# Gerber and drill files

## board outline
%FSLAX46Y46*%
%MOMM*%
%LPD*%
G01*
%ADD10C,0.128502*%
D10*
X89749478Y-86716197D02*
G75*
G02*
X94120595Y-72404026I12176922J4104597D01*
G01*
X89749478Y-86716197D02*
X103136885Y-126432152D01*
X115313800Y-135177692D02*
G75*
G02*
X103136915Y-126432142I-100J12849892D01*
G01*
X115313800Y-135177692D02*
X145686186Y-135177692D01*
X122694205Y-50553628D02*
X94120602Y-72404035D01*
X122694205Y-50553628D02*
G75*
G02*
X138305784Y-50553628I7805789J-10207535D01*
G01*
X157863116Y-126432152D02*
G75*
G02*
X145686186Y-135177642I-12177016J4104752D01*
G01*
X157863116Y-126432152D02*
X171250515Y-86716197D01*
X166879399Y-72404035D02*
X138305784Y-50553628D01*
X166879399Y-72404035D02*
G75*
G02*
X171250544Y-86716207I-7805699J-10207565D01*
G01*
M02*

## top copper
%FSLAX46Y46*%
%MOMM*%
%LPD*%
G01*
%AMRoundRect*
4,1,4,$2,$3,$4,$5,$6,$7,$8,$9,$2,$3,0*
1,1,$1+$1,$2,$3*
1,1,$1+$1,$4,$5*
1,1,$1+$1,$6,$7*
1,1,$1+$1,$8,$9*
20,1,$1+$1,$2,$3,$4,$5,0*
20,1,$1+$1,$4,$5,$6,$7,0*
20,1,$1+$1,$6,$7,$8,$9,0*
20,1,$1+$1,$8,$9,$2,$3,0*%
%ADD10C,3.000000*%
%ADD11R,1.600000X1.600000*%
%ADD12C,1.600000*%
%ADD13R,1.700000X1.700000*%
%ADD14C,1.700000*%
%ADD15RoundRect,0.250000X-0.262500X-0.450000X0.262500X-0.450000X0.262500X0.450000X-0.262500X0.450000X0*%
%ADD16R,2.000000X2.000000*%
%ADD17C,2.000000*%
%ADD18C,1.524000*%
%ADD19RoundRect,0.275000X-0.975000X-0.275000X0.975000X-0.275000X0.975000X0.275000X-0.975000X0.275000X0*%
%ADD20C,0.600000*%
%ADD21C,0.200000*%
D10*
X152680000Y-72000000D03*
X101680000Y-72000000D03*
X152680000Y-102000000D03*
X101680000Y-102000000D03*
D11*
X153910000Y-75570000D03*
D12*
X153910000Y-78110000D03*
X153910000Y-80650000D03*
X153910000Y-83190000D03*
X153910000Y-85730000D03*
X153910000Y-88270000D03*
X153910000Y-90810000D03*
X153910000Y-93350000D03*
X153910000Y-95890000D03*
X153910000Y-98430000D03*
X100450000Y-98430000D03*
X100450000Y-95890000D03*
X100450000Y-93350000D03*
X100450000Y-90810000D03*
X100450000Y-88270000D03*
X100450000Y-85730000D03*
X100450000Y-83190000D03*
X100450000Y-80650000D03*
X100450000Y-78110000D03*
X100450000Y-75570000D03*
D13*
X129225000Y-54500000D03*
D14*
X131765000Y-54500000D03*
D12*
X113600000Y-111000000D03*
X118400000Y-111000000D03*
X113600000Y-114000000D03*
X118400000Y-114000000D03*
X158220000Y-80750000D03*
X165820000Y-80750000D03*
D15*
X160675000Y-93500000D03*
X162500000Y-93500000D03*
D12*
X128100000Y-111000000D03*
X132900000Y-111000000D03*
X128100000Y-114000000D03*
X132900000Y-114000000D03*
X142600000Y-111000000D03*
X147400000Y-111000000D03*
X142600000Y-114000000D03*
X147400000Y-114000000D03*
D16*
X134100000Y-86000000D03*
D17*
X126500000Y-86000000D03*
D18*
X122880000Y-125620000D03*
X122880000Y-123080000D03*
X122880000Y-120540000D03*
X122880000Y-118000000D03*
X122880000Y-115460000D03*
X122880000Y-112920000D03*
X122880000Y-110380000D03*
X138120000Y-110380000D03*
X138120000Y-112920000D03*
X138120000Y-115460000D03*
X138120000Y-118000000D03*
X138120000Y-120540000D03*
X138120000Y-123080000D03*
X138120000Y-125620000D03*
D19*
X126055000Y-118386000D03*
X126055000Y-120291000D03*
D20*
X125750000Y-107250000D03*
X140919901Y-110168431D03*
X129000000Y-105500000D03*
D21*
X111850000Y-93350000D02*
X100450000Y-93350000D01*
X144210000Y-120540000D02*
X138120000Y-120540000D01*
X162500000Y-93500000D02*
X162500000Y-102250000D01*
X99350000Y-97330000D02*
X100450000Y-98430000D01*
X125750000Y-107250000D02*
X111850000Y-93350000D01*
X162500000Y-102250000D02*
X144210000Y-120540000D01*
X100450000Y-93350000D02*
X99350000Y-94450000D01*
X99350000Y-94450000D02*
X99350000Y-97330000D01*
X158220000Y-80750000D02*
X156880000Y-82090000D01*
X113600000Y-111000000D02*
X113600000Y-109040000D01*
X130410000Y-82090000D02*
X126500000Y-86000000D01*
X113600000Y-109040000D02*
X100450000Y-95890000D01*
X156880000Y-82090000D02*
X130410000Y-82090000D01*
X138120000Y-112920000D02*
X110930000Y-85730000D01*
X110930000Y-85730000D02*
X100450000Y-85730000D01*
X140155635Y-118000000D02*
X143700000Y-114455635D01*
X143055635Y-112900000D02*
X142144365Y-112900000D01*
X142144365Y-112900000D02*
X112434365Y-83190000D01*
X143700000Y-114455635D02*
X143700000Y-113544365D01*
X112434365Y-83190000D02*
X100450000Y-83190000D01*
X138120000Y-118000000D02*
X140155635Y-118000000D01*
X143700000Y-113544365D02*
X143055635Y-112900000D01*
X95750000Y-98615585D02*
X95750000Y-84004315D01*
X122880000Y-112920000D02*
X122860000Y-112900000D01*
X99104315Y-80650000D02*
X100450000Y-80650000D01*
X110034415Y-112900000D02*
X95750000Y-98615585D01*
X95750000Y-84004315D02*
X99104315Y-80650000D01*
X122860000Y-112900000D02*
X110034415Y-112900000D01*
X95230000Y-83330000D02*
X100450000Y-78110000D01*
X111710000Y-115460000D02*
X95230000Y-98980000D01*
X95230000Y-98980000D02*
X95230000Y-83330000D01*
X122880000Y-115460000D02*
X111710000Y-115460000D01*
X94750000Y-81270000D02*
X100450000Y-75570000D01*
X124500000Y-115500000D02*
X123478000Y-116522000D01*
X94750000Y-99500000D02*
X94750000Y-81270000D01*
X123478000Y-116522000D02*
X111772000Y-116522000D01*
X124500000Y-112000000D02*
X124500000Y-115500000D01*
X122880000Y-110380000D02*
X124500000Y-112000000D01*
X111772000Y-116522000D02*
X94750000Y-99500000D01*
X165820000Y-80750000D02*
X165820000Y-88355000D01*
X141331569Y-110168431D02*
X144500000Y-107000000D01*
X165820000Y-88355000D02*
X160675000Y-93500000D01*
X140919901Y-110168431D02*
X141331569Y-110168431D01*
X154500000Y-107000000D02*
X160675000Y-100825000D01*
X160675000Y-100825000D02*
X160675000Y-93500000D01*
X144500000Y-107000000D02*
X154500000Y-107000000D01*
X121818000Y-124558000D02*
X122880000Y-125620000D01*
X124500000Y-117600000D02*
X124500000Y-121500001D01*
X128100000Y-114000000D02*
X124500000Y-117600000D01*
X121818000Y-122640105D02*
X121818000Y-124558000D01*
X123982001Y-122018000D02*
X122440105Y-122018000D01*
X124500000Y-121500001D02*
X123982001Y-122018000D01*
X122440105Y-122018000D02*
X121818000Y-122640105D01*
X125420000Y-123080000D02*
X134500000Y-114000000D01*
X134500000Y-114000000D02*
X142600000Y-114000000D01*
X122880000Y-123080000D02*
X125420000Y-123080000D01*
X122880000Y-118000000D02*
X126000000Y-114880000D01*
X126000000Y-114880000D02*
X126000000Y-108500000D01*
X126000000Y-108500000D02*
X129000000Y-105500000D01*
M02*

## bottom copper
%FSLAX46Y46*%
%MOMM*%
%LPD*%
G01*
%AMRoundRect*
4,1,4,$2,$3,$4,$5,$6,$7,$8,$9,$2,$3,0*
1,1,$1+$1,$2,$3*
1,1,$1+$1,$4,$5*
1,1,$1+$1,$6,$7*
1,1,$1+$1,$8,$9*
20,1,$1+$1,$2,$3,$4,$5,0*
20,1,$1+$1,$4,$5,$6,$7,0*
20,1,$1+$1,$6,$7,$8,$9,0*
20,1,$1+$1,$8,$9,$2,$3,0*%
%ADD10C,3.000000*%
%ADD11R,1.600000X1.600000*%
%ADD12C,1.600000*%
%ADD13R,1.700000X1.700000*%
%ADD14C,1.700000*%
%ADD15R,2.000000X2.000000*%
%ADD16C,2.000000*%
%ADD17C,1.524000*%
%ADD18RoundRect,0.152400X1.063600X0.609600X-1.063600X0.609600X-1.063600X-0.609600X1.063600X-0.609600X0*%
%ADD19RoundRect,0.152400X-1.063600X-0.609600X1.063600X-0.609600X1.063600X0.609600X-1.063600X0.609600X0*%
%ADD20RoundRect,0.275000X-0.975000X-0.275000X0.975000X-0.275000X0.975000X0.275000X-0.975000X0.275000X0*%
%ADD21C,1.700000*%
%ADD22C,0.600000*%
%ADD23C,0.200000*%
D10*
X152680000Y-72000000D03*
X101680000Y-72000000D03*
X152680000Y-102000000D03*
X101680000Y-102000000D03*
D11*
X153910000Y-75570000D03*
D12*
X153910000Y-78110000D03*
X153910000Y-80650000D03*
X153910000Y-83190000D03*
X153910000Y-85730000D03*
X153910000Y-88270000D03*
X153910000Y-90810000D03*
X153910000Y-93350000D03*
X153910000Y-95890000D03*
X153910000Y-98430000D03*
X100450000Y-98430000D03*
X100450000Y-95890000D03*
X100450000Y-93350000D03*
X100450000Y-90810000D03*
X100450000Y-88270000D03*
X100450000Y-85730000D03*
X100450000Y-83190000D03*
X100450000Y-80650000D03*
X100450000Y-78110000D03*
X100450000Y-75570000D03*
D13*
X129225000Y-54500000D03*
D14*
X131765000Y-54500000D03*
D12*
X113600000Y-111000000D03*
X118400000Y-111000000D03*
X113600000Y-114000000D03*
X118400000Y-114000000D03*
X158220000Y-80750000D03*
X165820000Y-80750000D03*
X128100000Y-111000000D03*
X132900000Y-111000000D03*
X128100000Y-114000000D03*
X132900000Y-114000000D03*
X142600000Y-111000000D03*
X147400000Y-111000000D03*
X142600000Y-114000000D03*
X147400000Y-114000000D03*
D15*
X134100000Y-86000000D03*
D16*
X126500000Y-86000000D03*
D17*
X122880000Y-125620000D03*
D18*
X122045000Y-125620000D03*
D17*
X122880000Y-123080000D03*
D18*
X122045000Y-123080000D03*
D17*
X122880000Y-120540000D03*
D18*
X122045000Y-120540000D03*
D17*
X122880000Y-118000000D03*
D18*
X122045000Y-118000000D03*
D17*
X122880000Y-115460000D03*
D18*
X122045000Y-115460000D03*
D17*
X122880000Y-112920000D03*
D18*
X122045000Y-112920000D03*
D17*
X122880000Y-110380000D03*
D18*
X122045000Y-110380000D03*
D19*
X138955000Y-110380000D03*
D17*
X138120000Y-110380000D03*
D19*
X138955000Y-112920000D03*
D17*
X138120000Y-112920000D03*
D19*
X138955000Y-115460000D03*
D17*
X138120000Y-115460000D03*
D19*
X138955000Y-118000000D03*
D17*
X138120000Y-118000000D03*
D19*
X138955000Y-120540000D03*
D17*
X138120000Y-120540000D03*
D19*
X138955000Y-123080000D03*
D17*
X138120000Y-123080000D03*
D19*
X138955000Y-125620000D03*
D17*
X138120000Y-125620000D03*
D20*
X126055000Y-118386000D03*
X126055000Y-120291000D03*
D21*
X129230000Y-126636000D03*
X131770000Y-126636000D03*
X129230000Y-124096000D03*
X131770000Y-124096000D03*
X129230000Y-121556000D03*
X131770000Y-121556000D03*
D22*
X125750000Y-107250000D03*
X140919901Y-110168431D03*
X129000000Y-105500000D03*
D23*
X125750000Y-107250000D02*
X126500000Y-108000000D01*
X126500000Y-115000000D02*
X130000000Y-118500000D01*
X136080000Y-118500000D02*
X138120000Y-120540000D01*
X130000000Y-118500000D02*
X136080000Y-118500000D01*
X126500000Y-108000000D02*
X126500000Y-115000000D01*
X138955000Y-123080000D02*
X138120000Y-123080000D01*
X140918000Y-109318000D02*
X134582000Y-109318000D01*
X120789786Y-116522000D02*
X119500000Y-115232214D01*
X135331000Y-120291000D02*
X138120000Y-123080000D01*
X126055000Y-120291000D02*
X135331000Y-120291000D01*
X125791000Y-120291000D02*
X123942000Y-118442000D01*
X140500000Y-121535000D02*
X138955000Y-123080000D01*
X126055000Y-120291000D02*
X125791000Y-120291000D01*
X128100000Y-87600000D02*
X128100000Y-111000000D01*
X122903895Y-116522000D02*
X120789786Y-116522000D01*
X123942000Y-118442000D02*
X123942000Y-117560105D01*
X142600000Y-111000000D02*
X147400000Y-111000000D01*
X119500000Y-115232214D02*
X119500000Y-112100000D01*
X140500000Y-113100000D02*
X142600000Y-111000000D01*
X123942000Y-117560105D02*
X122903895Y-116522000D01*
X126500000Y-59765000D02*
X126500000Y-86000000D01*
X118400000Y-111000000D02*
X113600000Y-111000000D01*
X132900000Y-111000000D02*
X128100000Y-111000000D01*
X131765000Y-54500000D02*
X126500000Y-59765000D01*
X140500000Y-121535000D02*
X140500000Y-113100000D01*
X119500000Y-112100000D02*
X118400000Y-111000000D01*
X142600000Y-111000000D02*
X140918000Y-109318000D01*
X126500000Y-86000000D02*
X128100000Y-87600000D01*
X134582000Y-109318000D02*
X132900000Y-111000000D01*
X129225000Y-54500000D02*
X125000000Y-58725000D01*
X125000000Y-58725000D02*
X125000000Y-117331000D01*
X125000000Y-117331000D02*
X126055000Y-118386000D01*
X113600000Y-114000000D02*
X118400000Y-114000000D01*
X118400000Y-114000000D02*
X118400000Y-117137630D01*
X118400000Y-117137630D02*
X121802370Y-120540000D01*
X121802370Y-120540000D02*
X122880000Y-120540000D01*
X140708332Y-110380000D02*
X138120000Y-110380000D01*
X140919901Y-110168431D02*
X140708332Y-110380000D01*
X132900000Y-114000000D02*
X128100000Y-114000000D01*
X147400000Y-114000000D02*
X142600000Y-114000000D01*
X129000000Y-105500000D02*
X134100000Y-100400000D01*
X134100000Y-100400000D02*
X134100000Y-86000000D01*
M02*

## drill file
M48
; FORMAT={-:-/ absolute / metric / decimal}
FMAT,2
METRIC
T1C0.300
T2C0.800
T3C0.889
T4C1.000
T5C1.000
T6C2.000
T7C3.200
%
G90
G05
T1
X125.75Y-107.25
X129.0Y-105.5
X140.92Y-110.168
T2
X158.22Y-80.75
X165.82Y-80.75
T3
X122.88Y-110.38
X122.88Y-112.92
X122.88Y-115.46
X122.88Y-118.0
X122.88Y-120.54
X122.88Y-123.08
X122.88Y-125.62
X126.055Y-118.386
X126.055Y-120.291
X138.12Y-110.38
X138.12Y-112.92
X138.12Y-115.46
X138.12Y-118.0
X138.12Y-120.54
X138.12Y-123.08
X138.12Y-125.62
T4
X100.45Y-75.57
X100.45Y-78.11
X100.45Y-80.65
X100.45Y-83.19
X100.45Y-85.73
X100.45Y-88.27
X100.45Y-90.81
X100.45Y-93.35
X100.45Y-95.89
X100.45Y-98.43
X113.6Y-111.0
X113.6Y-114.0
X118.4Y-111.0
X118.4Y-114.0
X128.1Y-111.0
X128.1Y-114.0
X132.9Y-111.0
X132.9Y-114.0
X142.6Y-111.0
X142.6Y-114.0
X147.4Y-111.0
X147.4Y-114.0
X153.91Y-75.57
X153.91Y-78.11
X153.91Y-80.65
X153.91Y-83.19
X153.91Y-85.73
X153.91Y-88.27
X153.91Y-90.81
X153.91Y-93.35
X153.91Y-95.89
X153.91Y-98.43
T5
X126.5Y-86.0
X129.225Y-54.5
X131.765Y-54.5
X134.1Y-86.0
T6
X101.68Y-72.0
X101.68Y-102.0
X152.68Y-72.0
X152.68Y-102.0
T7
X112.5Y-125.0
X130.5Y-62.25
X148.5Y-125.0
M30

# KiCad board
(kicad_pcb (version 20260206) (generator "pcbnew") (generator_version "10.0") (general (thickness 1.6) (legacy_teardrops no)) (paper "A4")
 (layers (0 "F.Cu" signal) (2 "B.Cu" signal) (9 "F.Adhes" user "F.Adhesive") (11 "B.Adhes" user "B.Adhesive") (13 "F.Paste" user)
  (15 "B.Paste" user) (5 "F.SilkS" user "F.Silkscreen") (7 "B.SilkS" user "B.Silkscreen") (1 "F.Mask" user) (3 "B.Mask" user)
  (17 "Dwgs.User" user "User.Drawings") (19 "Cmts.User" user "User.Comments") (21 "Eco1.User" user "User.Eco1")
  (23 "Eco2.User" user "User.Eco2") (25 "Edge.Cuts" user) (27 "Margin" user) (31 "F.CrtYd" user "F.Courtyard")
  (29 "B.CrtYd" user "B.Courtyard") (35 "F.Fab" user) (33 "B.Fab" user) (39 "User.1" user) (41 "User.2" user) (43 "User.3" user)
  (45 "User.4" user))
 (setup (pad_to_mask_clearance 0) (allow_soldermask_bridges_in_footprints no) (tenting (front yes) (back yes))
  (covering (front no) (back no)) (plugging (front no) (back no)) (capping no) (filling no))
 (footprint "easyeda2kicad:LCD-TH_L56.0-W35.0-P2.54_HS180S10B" (layer "F.Cu") (at 127.18 87 -90)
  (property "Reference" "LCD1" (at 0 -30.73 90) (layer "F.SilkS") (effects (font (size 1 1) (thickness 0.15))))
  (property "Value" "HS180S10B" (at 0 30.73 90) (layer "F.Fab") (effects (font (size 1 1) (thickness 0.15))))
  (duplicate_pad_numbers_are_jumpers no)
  (pad "" thru_hole circle (at -15 -25.5 270) (size 3 3) (drill 2) (layers "*.Cu" "*.Mask") (remove_unused_layers no))
  (pad "" thru_hole circle (at -15 25.5 270) (size 3 3) (drill 2) (layers "*.Cu" "*.Mask") (remove_unused_layers no))
  (pad "" thru_hole circle (at 15 -25.5 270) (size 3 3) (drill 2) (layers "*.Cu" "*.Mask") (remove_unused_layers no))
  (pad "" thru_hole circle (at 15 25.5 270) (size 3 3) (drill 2) (layers "*.Cu" "*.Mask") (remove_unused_layers no))
  (pad "1" thru_hole rect (at -11.43 -26.73 270) (size 1.6 1.6) (drill 0.999998) (layers "*.Cu" "*.Mask") (remove_unused_layers no)
   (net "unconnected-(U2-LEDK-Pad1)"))
  (pad "2" thru_hole circle (at -8.89 -26.73 270) (size 1.6 1.6) (drill 0.999998) (layers "*.Cu" "*.Mask") (remove_unused_layers no)
   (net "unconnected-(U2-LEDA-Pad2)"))
  (pad "3" thru_hole circle (at -6.35 -26.73 270) (size 1.6 1.6) (drill 0.999998) (layers "*.Cu" "*.Mask") (remove_unused_layers no)
   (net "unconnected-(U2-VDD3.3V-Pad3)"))
  (pad "4" thru_hole circle (at -3.81 -26.73 270) (size 1.6 1.6) (drill 0.999998) (layers "*.Cu" "*.Mask") (remove_unused_layers no)
   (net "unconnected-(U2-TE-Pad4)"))
  (pad "5" thru_hole circle (at -1.27 -26.73 270) (size 1.6 1.6) (drill 0.999998) (layers "*.Cu" "*.Mask") (remove_unused_layers no)
   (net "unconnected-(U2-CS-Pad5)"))
  (pad "6" thru_hole circle (at 1.27 -26.73 270) (size 1.6 1.6) (drill 0.999998) (layers "*.Cu" "*.Mask") (remove_unused_layers no)
   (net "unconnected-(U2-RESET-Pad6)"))
  (pad "7" thru_hole circle (at 3.81 -26.73 270) (size 1.6 1.6) (drill 0.999998) (layers "*.Cu" "*.Mask") (remove_unused_layers no)
   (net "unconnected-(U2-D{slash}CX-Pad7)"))
  (pad "8" thru_hole circle (at 6.35 -26.73 270) (size 1.6 1.6) (drill 0.999998) (layers "*.Cu" "*.Mask") (remove_unused_layers no)
   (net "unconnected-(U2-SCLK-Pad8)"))
  (pad "9" thru_hole circle (at 8.89 -26.73 270) (size 1.6 1.6) (drill 0.999998) (layers "*.Cu" "*.Mask") (remove_unused_layers no)
   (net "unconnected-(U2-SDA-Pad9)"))
  (pad "10" thru_hole circle (at 11.43 -26.73 270) (size 1.6 1.6) (drill 0.999998) (layers "*.Cu" "*.Mask") (remove_unused_layers no)
   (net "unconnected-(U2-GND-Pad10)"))
  (pad "11" thru_hole circle (at 11.43 26.73 270) (size 1.6 1.6) (drill 0.999998) (layers "*.Cu" "*.Mask") (remove_unused_layers no)
   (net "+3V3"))
  (pad "12" thru_hole circle (at 8.89 26.73 270) (size 1.6 1.6) (drill 0.999998) (layers "*.Cu" "*.Mask") (remove_unused_layers no)
   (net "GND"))
  (pad "13" thru_hole circle (at 6.35 26.73 270) (size 1.6 1.6) (drill 0.999998) (layers "*.Cu" "*.Mask") (remove_unused_layers no)
   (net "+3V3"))
  (pad "14" thru_hole circle (at 3.81 26.73 270) (size 1.6 1.6) (drill 0.999998) (layers "*.Cu" "*.Mask") (remove_unused_layers no))
  (pad "15" thru_hole circle (at 1.27 26.73 270) (size 1.6 1.6) (drill 0.999998) (layers "*.Cu" "*.Mask") (remove_unused_layers no))
  (pad "16" thru_hole circle (at -1.27 26.73 270) (size 1.6 1.6) (drill 0.999998) (layers "*.Cu" "*.Mask") (remove_unused_layers no)
   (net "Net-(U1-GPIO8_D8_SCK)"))
  (pad "17" thru_hole circle (at -3.81 26.73 270) (size 1.6 1.6) (drill 0.999998) (layers "*.Cu" "*.Mask") (remove_unused_layers no)
   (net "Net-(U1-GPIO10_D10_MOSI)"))
  (pad "18" thru_hole circle (at -6.35 26.73 270) (size 1.6 1.6) (drill 0.999998) (layers "*.Cu" "*.Mask") (remove_unused_layers no)
   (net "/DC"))
  (pad "19" thru_hole circle (at -8.89 26.73 270) (size 1.6 1.6) (drill 0.999998) (layers "*.Cu" "*.Mask") (remove_unused_layers no)
   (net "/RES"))
  (pad "20" thru_hole circle (at -11.43 26.73 270) (size 1.6 1.6) (drill 0.999998) (layers "*.Cu" "*.Mask") (remove_unused_layers no)
   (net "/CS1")))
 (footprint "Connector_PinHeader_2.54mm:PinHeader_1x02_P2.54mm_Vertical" (layer "F.Cu") (at 129.225 54.5 90)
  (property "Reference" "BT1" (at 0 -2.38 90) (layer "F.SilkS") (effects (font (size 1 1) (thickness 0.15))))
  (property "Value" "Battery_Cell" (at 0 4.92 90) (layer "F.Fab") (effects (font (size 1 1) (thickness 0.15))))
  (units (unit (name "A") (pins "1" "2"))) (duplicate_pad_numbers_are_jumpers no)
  (pad "1" thru_hole rect (at 0 0 90) (size 1.7 1.7) (drill 1) (layers "*.Cu" "*.Mask") (remove_unused_layers no) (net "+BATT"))
  (pad "2" thru_hole circle (at 0 2.54 90) (size 1.7 1.7) (drill 1) (layers "*.Cu" "*.Mask") (remove_unused_layers no) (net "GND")))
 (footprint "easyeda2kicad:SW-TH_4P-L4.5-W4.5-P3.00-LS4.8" (layer "F.Cu") (at 116 112.5)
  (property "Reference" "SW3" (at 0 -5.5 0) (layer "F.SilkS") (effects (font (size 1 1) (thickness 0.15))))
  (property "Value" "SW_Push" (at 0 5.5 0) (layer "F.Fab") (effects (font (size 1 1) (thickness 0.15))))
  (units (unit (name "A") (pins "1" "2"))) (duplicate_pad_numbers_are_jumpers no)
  (pad "1" thru_hole circle (at -2.4 -1.5) (size 1.6 1.6) (drill 0.999998) (layers "*.Cu" "*.Mask") (remove_unused_layers no) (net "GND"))
  (pad "1" thru_hole circle (at 2.4 -1.5) (size 1.6 1.6) (drill 0.999998) (layers "*.Cu" "*.Mask") (remove_unused_layers no) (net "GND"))
  (pad "2" thru_hole circle (at -2.4 1.5) (size 1.6 1.6) (drill 0.999998) (layers "*.Cu" "*.Mask") (remove_unused_layers no)
   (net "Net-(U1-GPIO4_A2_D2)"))
  (pad "2" thru_hole circle (at 2.4 1.5) (size 1.6 1.6) (drill 0.999998) (layers "*.Cu" "*.Mask") (remove_unused_layers no)
   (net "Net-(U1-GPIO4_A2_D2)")))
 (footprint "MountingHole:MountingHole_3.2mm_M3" (layer "F.Cu") (at 112.5 125)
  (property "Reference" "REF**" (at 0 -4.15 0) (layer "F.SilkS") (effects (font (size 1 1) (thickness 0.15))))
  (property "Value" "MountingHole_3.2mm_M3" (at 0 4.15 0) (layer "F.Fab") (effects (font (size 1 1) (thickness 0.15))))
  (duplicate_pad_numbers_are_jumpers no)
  (pad "" np_thru_hole circle (at 0 0) (size 3.2 3.2) (drill 3.2) (layers "*.Cu" "*.Mask")))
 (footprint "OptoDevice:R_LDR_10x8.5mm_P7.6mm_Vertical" (layer "F.Cu") (at 158.22 80.75)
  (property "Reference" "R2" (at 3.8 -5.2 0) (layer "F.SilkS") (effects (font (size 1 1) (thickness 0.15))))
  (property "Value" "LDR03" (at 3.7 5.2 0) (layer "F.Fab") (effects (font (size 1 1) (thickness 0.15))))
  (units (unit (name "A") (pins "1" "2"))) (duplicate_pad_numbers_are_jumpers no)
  (pad "1" thru_hole circle (at 0 0) (size 1.6 1.6) (drill 0.8) (layers "*.Cu" "*.Mask") (remove_unused_layers no) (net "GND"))
  (pad "2" thru_hole circle (at 7.6 0) (size 1.6 1.6) (drill 0.8) (layers "*.Cu" "*.Mask") (remove_unused_layers no)
   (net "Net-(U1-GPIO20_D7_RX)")))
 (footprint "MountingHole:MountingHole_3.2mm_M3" (layer "F.Cu") (at 148.5 125)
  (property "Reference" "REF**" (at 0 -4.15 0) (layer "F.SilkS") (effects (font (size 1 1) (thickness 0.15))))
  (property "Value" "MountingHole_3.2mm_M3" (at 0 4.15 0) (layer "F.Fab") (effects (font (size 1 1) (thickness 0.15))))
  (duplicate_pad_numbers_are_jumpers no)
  (pad "" np_thru_hole circle (at 0 0) (size 3.2 3.2) (drill 3.2) (layers "*.Cu" "*.Mask")))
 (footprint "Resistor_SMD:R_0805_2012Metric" (layer "F.Cu") (at 161.5875 93.5)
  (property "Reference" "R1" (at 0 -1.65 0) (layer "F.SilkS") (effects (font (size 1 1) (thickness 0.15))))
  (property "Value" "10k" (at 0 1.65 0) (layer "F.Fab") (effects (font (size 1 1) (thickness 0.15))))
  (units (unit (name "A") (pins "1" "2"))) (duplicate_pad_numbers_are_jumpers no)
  (pad "1" smd roundrect (at -0.9125 0) (size 1.025 1.4) (layers "F.Cu" "F.Mask" "F.Paste") (roundrect_rratio 0.243902)
   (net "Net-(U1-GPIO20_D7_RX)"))
  (pad "2" smd roundrect (at 0.9125 0) (size 1.025 1.4) (layers "F.Cu" "F.Mask" "F.Paste") (roundrect_rratio 0.243902) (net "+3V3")))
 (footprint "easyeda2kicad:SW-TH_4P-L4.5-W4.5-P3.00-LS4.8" (layer "F.Cu") (at 130.5 112.5)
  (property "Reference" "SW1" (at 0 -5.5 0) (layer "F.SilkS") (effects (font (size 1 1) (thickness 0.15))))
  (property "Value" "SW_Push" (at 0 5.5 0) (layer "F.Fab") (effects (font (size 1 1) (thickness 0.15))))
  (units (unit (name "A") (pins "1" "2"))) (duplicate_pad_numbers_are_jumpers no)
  (pad "1" thru_hole circle (at -2.4 -1.5) (size 1.6 1.6) (drill 0.999998) (layers "*.Cu" "*.Mask") (remove_unused_layers no) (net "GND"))
  (pad "1" thru_hole circle (at 2.4 -1.5) (size 1.6 1.6) (drill 0.999998) (layers "*.Cu" "*.Mask") (remove_unused_layers no) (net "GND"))
  (pad "2" thru_hole circle (at -2.4 1.5) (size 1.6 1.6) (drill 0.999998) (layers "*.Cu" "*.Mask") (remove_unused_layers no)
   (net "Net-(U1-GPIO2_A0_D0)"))
  (pad "2" thru_hole circle (at 2.4 1.5) (size 1.6 1.6) (drill 0.999998) (layers "*.Cu" "*.Mask") (remove_unused_layers no)
   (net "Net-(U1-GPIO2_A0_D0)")))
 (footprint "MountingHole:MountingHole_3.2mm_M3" (layer "F.Cu") (at 130.5 62.25)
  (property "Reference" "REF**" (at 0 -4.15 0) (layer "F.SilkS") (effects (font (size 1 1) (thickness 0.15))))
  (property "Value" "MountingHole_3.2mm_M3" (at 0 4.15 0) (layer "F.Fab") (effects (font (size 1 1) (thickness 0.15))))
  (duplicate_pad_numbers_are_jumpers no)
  (pad "" np_thru_hole circle (at 0 0) (size 3.2 3.2) (drill 3.2) (layers "*.Cu" "*.Mask")))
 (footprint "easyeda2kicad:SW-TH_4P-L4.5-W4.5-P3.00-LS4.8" (layer "F.Cu") (at 145 112.5)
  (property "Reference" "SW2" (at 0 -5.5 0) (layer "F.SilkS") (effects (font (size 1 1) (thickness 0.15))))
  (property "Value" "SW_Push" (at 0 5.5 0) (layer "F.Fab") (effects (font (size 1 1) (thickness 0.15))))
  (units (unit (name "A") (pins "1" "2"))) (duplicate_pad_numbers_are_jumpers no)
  (pad "1" thru_hole circle (at -2.4 -1.5) (size 1.6 1.6) (drill 0.999998) (layers "*.Cu" "*.Mask") (remove_unused_layers no) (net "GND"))
  (pad "1" thru_hole circle (at 2.4 -1.5) (size 1.6 1.6) (drill 0.999998) (layers "*.Cu" "*.Mask") (remove_unused_layers no) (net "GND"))
  (pad "2" thru_hole circle (at -2.4 1.5) (size 1.6 1.6) (drill 0.999998) (layers "*.Cu" "*.Mask") (remove_unused_layers no)
   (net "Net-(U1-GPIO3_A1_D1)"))
  (pad "2" thru_hole circle (at 2.4 1.5) (size 1.6 1.6) (drill 0.999998) (layers "*.Cu" "*.Mask") (remove_unused_layers no)
   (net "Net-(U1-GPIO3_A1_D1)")))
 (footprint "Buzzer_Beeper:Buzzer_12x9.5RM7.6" (layer "B.Cu") (at 134.1 86 180)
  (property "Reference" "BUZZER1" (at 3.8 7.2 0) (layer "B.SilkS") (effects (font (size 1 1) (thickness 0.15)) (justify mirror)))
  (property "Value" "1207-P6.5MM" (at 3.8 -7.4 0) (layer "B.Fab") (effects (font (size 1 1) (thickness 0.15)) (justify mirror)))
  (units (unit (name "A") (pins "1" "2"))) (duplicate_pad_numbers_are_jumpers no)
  (pad "1" thru_hole rect (at 0 0 180) (size 2 2) (drill 1) (layers "*.Cu" "*.Mask") (remove_unused_layers no) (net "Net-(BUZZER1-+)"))
  (pad "2" thru_hole circle (at 7.6 0 180) (size 2 2) (drill 1) (layers "*.Cu" "*.Mask") (remove_unused_layers no) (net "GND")))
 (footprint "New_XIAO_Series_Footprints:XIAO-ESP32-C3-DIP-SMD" (layer "B.Cu") (at 130.5 118 -90)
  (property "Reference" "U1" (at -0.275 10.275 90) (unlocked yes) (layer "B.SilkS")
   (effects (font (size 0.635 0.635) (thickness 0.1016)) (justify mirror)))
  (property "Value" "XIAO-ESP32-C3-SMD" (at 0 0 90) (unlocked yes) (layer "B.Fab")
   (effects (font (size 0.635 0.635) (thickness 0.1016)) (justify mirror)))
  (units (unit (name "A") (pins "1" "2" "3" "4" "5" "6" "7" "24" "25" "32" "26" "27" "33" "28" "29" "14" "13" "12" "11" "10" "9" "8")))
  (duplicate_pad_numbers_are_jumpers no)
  (pad "1" thru_hole circle (at 7.62 7.62 180) (size 1.524 1.524) (drill 0.889) (layers "*.Cu" "*.Mask") (remove_unused_layers no)
   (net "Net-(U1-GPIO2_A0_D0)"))
  (pad "1" smd roundrect (at 7.62 8.455 180) (size 2.432 1.524) (layers "B.Cu" "B.Mask") (roundrect_rratio 0.1) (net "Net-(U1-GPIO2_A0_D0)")
   (thermal_bridge_angle 45))
  (pad "2" thru_hole circle (at 5.08 7.62 180) (size 1.524 1.524) (drill 0.889) (layers "*.Cu" "*.Mask") (remove_unused_layers no)
   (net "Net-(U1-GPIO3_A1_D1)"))
  (pad "2" smd roundrect (at 5.08 8.455 180) (size 2.432 1.524) (layers "B.Cu" "B.Mask") (roundrect_rratio 0.1) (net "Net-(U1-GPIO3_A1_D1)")
   (thermal_bridge_angle 45))
  (pad "3" thru_hole circle (at 2.54 7.62 180) (size 1.524 1.524) (drill 0.889) (layers "*.Cu" "*.Mask") (remove_unused_layers no)
   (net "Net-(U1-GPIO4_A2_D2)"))
  (pad "3" smd roundrect (at 2.54 8.455 180) (size 2.432 1.524) (layers "B.Cu" "B.Mask") (roundrect_rratio 0.1) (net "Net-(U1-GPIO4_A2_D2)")
   (thermal_bridge_angle 45))
  (pad "4" thru_hole circle (at 0 7.62 180) (size 1.524 1.524) (drill 0.889) (layers "*.Cu" "*.Mask") (remove_unused_layers no)
   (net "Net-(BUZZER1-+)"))
  (pad "4" smd roundrect (at 0 8.455 180) (size 2.432 1.524) (layers "B.Cu" "B.Mask") (roundrect_rratio 0.1) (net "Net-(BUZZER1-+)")
   (thermal_bridge_angle 45))
  (pad "5" thru_hole circle (at -2.54 7.62 180) (size 1.524 1.524) (drill 0.889) (layers "*.Cu" "*.Mask") (remove_unused_layers no)
   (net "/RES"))
  (pad "5" smd roundrect (at -2.54 8.455 180) (size 2.432 1.524) (layers "B.Cu" "B.Mask") (roundrect_rratio 0.1) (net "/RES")
   (thermal_bridge_angle 45))
  (pad "6" thru_hole circle (at -5.08 7.62 180) (size 1.524 1.524) (drill 0.889) (layers "*.Cu" "*.Mask") (remove_unused_layers no)
   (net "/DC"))
  (pad "6" smd roundrect (at -5.08 8.455 180) (size 2.432 1.524) (layers "B.Cu" "B.Mask") (roundrect_rratio 0.1) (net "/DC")
   (thermal_bridge_angle 45))
  (pad "7" thru_hole circle (at -7.62 7.62 180) (size 1.524 1.524) (drill 0.889) (layers "*.Cu" "*.Mask") (remove_unused_layers no)
   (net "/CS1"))
  (pad "7" smd roundrect (at -7.62 8.455 180) (size 2.432 1.524) (layers "B.Cu" "B.Mask") (roundrect_rratio 0.1) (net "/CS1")
   (thermal_bridge_angle 45))
  (pad "8" smd roundrect (at -7.62 -8.455) (size 2.432 1.524) (layers "B.Cu" "B.Mask") (roundrect_rratio 0.1) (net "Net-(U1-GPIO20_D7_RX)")
   (thermal_bridge_angle 45))
  (pad "8" thru_hole circle (at -7.62 -7.62) (size 1.524 1.524) (drill 0.889) (layers "*.Cu" "*.Mask") (remove_unused_layers no)
   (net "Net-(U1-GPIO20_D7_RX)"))
  (pad "9" smd roundrect (at -5.08 -8.455) (size 2.432 1.524) (layers "B.Cu" "B.Mask") (roundrect_rratio 0.1) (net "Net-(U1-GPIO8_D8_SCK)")
   (thermal_bridge_angle 45))
  (pad "9" thru_hole circle (at -5.08 -7.62) (size 1.524 1.524) (drill 0.889) (layers "*.Cu" "*.Mask") (remove_unused_layers no)
   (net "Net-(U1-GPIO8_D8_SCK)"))
  (pad "10" smd roundrect (at -2.54 -8.455) (size 2.432 1.524) (layers "B.Cu" "B.Mask") (roundrect_rratio 0.1)
   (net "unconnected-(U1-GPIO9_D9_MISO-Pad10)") (thermal_bridge_angle 45))
  (pad "10" thru_hole circle (at -2.54 -7.62) (size 1.524 1.524) (drill 0.889) (layers "*.Cu" "*.Mask") (remove_unused_layers no)
   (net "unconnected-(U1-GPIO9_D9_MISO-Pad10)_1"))
  (pad "11" smd roundrect (at 0 -8.455) (size 2.432 1.524) (layers "B.Cu" "B.Mask") (roundrect_rratio 0.1) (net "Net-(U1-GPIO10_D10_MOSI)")
   (thermal_bridge_angle 45))
  (pad "11" thru_hole circle (at 0 -7.62) (size 1.524 1.524) (drill 0.889) (layers "*.Cu" "*.Mask") (remove_unused_layers no)
   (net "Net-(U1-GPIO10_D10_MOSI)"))
  (pad "12" smd roundrect (at 2.54 -8.455) (size 2.432 1.524) (layers "B.Cu" "B.Mask") (roundrect_rratio 0.1) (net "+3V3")
   (thermal_bridge_angle 45))
  (pad "12" thru_hole circle (at 2.54 -7.62) (size 1.524 1.524) (drill 0.889) (layers "*.Cu" "*.Mask") (remove_unused_layers no)
   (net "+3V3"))
  (pad "13" smd roundrect (at 5.08 -8.455) (size 2.432 1.524) (layers "B.Cu" "B.Mask") (roundrect_rratio 0.1) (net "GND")
   (thermal_bridge_angle 45))
  (pad "13" thru_hole circle (at 5.08 -7.62) (size 1.524 1.524) (drill 0.889) (layers "*.Cu" "*.Mask") (remove_unused_layers no) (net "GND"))
  (pad "14" smd roundrect (at 7.62 -8.455) (size 2.432 1.524) (layers "B.Cu" "B.Mask") (roundrect_rratio 0.1) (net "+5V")
   (thermal_bridge_angle 45))
  (pad "14" thru_hole circle (at 7.62 -7.62) (size 1.524 1.524) (drill 0.889) (layers "*.Cu" "*.Mask") (remove_unused_layers no) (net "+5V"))
  (pad "15" thru_hole roundrect (at 0.386 4.445) (size 2.5 1.1) (drill 0.889) (layers "*.Cu" "*.Mask") (remove_unused_layers no)
   (roundrect_rratio 0.25) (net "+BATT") (thermal_bridge_angle 45))
  (pad "16" thru_hole roundrect (at 2.291 4.445) (size 2.5 1.1) (drill 0.889) (layers "*.Cu" "*.Mask") (remove_unused_layers no)
   (roundrect_rratio 0.25) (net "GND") (thermal_bridge_angle 45))
  (pad "17" smd circle (at 8.636 1.27) (size 1.7 1.7) (layers "B.Cu" "B.Mask" "B.Paste"))
  (pad "18" smd circle (at 8.636 -1.27) (size 1.7 1.7) (layers "B.Cu" "B.Mask" "B.Paste"))
  (pad "19" smd circle (at 6.096 1.27) (size 1.7 1.7) (layers "B.Cu" "B.Mask" "B.Paste"))
  (pad "20" smd circle (at 6.096 -1.27) (size 1.7 1.7) (layers "B.Cu" "B.Mask" "B.Paste"))
  (pad "21" smd circle (at 3.556 1.27) (size 1.7 1.7) (layers "B.Cu" "B.Mask" "B.Paste"))
  (pad "22" smd circle (at 3.556 -1.27) (size 1.7 1.7) (layers "B.Cu" "B.Mask" "B.Paste")))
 (gr_arc (start 89.749478 86.716197) (mid 89.636692 78.858169) (end 94.120602 72.404035) (stroke (width 0.128502) (type default))
  (layer "Edge.Cuts"))
 (gr_line (start 89.749478 86.716197) (end 103.136885 126.432152) (stroke (width 0.128502) (type default)) (layer "Edge.Cuts"))
 (gr_arc (start 115.3138 135.177692) (mid 107.817744 132.764785) (end 103.136885 126.432152) (stroke (width 0.128502) (type default))
  (layer "Edge.Cuts"))
 (gr_line (start 115.3138 135.177692) (end 145.686186 135.177692) (stroke (width 0.128502) (type default)) (layer "Edge.Cuts"))
 (gr_line (start 122.694205 50.553628) (end 94.120602 72.404035) (stroke (width 0.128502) (type default)) (layer "Edge.Cuts"))
 (gr_arc (start 122.694205 50.553628) (mid 130.499996 47.9111) (end 138.305784 50.553628) (stroke (width 0.128502) (type default))
  (layer "Edge.Cuts"))
 (gr_arc (start 157.863116 126.432152) (mid 153.182199 132.764729) (end 145.686186 135.177692) (stroke (width 0.128502) (type default))
  (layer "Edge.Cuts"))
 (gr_line (start 157.863116 126.432152) (end 171.250515 86.716197) (stroke (width 0.128502) (type default)) (layer "Edge.Cuts"))
 (gr_line (start 166.879399 72.404035) (end 138.305784 50.553628) (stroke (width 0.128502) (type default)) (layer "Edge.Cuts"))
 (gr_arc (start 166.879399 72.404035) (mid 171.363322 78.858174) (end 171.250515 86.716197) (stroke (width 0.128502) (type default))
  (layer "Edge.Cuts"))
 (segment (start 111.85 93.35) (end 100.45 93.35) (width 0.2) (layer "F.Cu") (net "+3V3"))
 (segment (start 144.21 120.54) (end 138.12 120.54) (width 0.2) (layer "F.Cu") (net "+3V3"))
 (segment (start 162.5 93.5) (end 162.5 102.25) (width 0.2) (layer "F.Cu") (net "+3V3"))
 (segment (start 99.35 97.33) (end 100.45 98.43) (width 0.2) (layer "F.Cu") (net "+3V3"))
 (segment (start 125.75 107.25) (end 111.85 93.35) (width 0.2) (layer "F.Cu") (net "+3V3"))
 (segment (start 162.5 102.25) (end 144.21 120.54) (width 0.2) (layer "F.Cu") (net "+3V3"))
 (segment (start 100.45 93.35) (end 99.35 94.45) (width 0.2) (layer "F.Cu") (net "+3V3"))
 (segment (start 99.35 94.45) (end 99.35 97.33) (width 0.2) (layer "F.Cu") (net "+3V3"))
 (via (at 125.75 107.25) (size 0.6) (drill 0.3) (layers "F.Cu" "B.Cu") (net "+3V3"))
 (segment (start 125.75 107.25) (end 126.5 108) (width 0.2) (layer "B.Cu") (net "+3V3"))
 (segment (start 126.5 115) (end 130 118.5) (width 0.2) (layer "B.Cu") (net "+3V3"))
 (segment (start 136.08 118.5) (end 138.12 120.54) (width 0.2) (layer "B.Cu") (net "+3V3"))
 (segment (start 130 118.5) (end 136.08 118.5) (width 0.2) (layer "B.Cu") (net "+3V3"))
 (segment (start 126.5 108) (end 126.5 115) (width 0.2) (layer "B.Cu") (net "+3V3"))
 (segment (start 158.22 80.75) (end 156.88 82.09) (width 0.2) (layer "F.Cu") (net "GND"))
 (segment (start 113.6 111) (end 113.6 109.04) (width 0.2) (layer "F.Cu") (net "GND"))
 (segment (start 130.41 82.09) (end 126.5 86) (width 0.2) (layer "F.Cu") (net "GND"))
 (segment (start 113.6 109.04) (end 100.45 95.89) (width 0.2) (layer "F.Cu") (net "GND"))
 (segment (start 156.88 82.09) (end 130.41 82.09) (width 0.2) (layer "F.Cu") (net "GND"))
 (segment (start 138.955 123.08) (end 138.12 123.08) (width 0.2) (layer "B.Cu") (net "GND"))
 (segment (start 140.918 109.318) (end 134.582 109.318) (width 0.2) (layer "B.Cu") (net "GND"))
 (segment (start 120.789786 116.522) (end 119.5 115.232214) (width 0.2) (layer "B.Cu") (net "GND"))
 (segment (start 135.331 120.291) (end 138.12 123.08) (width 0.2) (layer "B.Cu") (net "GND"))
 (segment (start 126.055 120.291) (end 135.331 120.291) (width 0.2) (layer "B.Cu") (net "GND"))
 (segment (start 125.791 120.291) (end 123.942 118.442) (width 0.2) (layer "B.Cu") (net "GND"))
 (segment (start 140.5 121.535) (end 138.955 123.08) (width 0.2) (layer "B.Cu") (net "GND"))
 (segment (start 126.055 120.291) (end 125.791 120.291) (width 0.2) (layer "B.Cu") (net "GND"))
 (segment (start 128.1 87.6) (end 128.1 111) (width 0.2) (layer "B.Cu") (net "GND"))
 (segment (start 122.903895 116.522) (end 120.789786 116.522) (width 0.2) (layer "B.Cu") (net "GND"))
 (segment (start 123.942 118.442) (end 123.942 117.560105) (width 0.2) (layer "B.Cu") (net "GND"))
 (segment (start 142.6 111) (end 147.4 111) (width 0.2) (layer "B.Cu") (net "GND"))
 (segment (start 119.5 115.232214) (end 119.5 112.1) (width 0.2) (layer "B.Cu") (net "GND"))
 (segment (start 140.5 113.1) (end 142.6 111) (width 0.2) (layer "B.Cu") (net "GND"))
 (segment (start 123.942 117.560105) (end 122.903895 116.522) (width 0.2) (layer "B.Cu") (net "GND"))
 (segment (start 126.5 59.765) (end 126.5 86) (width 0.2) (layer "B.Cu") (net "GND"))
 (segment (start 118.4 111) (end 113.6 111) (width 0.2) (layer "B.Cu") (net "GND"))
 (segment (start 132.9 111) (end 128.1 111) (width 0.2) (layer "B.Cu") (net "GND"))
 (segment (start 131.765 54.5) (end 126.5 59.765) (width 0.2) (layer "B.Cu") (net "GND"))
 (segment (start 140.5 121.535) (end 140.5 113.1) (width 0.2) (layer "B.Cu") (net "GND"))
 (segment (start 119.5 112.1) (end 118.4 111) (width 0.2) (layer "B.Cu") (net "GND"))
 (segment (start 142.6 111) (end 140.918 109.318) (width 0.2) (layer "B.Cu") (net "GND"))
 (segment (start 126.5 86) (end 128.1 87.6) (width 0.2) (layer "B.Cu") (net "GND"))
 (segment (start 134.582 109.318) (end 132.9 111) (width 0.2) (layer "B.Cu") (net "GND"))
 (segment (start 138.12 112.92) (end 110.93 85.73) (width 0.2) (layer "F.Cu") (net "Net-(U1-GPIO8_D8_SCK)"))
 (segment (start 110.93 85.73) (end 100.45 85.73) (width 0.2) (layer "F.Cu") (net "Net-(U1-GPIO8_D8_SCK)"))
 (segment (start 140.155635 118) (end 143.7 114.455635) (width 0.2) (layer "F.Cu") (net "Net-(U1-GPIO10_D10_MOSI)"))
 (segment (start 143.055635 112.9) (end 142.144365 112.9) (width 0.2) (layer "F.Cu") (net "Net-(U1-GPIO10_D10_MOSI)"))
 (segment (start 142.144365 112.9) (end 112.434365 83.19) (width 0.2) (layer "F.Cu") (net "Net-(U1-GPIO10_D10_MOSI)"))
 (segment (start 143.7 114.455635) (end 143.7 113.544365) (width 0.2) (layer "F.Cu") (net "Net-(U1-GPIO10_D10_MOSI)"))
 (segment (start 112.434365 83.19) (end 100.45 83.19) (width 0.2) (layer "F.Cu") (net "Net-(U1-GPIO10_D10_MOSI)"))
 (segment (start 138.12 118) (end 140.155635 118) (width 0.2) (layer "F.Cu") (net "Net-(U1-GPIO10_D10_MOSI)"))
 (segment (start 143.7 113.544365) (end 143.055635 112.9) (width 0.2) (layer "F.Cu") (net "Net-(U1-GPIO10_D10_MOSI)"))
 (segment (start 95.75 98.615585) (end 95.75 84.004315) (width 0.2) (layer "F.Cu") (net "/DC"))
 (segment (start 122.88 112.92) (end 122.86 112.9) (width 0.2) (layer "F.Cu") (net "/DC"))
 (segment (start 99.104315 80.65) (end 100.45 80.65) (width 0.2) (layer "F.Cu") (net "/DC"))
 (segment (start 110.034415 112.9) (end 95.75 98.615585) (width 0.2) (layer "F.Cu") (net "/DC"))
 (segment (start 95.75 84.004315) (end 99.104315 80.65) (width 0.2) (layer "F.Cu") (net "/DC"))
 (segment (start 122.86 112.9) (end 110.034415 112.9) (width 0.2) (layer "F.Cu") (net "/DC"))
 (segment (start 95.23 83.33) (end 100.45 78.11) (width 0.2) (layer "F.Cu") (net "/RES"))
 (segment (start 111.71 115.46) (end 95.23 98.98) (width 0.2) (layer "F.Cu") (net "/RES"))
 (segment (start 95.23 98.98) (end 95.23 83.33) (width 0.2) (layer "F.Cu") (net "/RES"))
 (segment (start 122.88 115.46) (end 111.71 115.46) (width 0.2) (layer "F.Cu") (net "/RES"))
 (segment (start 94.75 81.27) (end 100.45 75.57) (width 0.2) (layer "F.Cu") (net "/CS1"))
 (segment (start 124.5 115.5) (end 123.478 116.522) (width 0.2) (layer "F.Cu") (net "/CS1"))
 (segment (start 94.75 99.5) (end 94.75 81.27) (width 0.2) (layer "F.Cu") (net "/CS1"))
 (segment (start 123.478 116.522) (end 111.772 116.522) (width 0.2) (layer "F.Cu") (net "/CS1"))
 (segment (start 124.5 112) (end 124.5 115.5) (width 0.2) (layer "F.Cu") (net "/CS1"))
 (segment (start 122.88 110.38) (end 124.5 112) (width 0.2) (layer "F.Cu") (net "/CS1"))
 (segment (start 111.772 116.522) (end 94.75 99.5) (width 0.2) (layer "F.Cu") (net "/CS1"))
 (segment (start 129.225 54.5) (end 125 58.725) (width 0.2) (layer "B.Cu") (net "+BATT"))
 (segment (start 125 58.725) (end 125 117.331) (width 0.2) (layer "B.Cu") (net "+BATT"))
 (segment (start 125 117.331) (end 126.055 118.386) (width 0.2) (layer "B.Cu") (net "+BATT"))
 (segment (start 113.6 114) (end 118.4 114) (width 0.2) (layer "B.Cu") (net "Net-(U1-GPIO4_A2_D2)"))
 (segment (start 118.4 114) (end 118.4 117.13763) (width 0.2) (layer "B.Cu") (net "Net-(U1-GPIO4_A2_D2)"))
 (segment (start 118.4 117.13763) (end 121.80237 120.54) (width 0.2) (layer "B.Cu") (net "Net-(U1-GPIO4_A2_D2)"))
 (segment (start 121.80237 120.54) (end 122.88 120.54) (width 0.2) (layer "B.Cu") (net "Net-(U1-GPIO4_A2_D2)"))
 (segment (start 165.82 80.75) (end 165.82 88.355) (width 0.2) (layer "F.Cu") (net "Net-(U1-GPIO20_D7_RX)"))
 (segment (start 141.331569 110.168431) (end 144.5 107) (width 0.2) (layer "F.Cu") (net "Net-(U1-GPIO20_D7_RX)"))
 (segment (start 165.82 88.355) (end 160.675 93.5) (width 0.2) (layer "F.Cu") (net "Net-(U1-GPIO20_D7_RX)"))
 (segment (start 140.919901 110.168431) (end 141.331569 110.168431) (width 0.2) (layer "F.Cu") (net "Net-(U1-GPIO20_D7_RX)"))
 (segment (start 154.5 107) (end 160.675 100.825) (width 0.2) (layer "F.Cu") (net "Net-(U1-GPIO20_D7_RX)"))
 (segment (start 160.675 100.825) (end 160.675 93.5) (width 0.2) (layer "F.Cu") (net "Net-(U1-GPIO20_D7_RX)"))
 (segment (start 144.5 107) (end 154.5 107) (width 0.2) (layer "F.Cu") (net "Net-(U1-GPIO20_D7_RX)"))
 (via (at 140.919901 110.168431) (size 0.6) (drill 0.3) (layers "F.Cu" "B.Cu") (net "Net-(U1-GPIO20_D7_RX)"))
 (segment (start 140.708332 110.38) (end 138.12 110.38) (width 0.2) (layer "B.Cu") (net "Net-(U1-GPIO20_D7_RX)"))
 (segment (start 140.919901 110.168431) (end 140.708332 110.38) (width 0.2) (layer "B.Cu") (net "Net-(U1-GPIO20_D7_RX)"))
 (segment (start 121.818 124.558) (end 122.88 125.62) (width 0.2) (layer "F.Cu") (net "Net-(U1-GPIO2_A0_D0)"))
 (segment (start 124.5 117.6) (end 124.5 121.500001) (width 0.2) (layer "F.Cu") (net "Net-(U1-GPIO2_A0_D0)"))
 (segment (start 128.1 114) (end 124.5 117.6) (width 0.2) (layer "F.Cu") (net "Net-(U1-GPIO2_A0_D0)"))
 (segment (start 121.818 122.640105) (end 121.818 124.558) (width 0.2) (layer "F.Cu") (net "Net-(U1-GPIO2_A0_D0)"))
 (segment (start 123.982001 122.018) (end 122.440105 122.018) (width 0.2) (layer "F.Cu") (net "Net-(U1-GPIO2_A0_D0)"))
 (segment (start 124.5 121.500001) (end 123.982001 122.018) (width 0.2) (layer "F.Cu") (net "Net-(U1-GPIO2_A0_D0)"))
 (segment (start 122.440105 122.018) (end 121.818 122.640105) (width 0.2) (layer "F.Cu") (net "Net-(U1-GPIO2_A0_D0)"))
 (segment (start 132.9 114) (end 128.1 114) (width 0.2) (layer "B.Cu") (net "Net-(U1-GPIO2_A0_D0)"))
 (segment (start 125.42 123.08) (end 134.5 114) (width 0.2) (layer "F.Cu") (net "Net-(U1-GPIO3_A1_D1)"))
 (segment (start 134.5 114) (end 142.6 114) (width 0.2) (layer "F.Cu") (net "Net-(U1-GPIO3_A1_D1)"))
 (segment (start 122.88 123.08) (end 125.42 123.08) (width 0.2) (layer "F.Cu") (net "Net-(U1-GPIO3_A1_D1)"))
 (segment (start 147.4 114) (end 142.6 114) (width 0.2) (layer "B.Cu") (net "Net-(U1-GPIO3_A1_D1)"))
 (segment (start 122.88 118) (end 126 114.88) (width 0.2) (layer "F.Cu") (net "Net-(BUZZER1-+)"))
 (segment (start 126 114.88) (end 126 108.5) (width 0.2) (layer "F.Cu") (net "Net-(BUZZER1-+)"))
 (segment (start 126 108.5) (end 129 105.5) (width 0.2) (layer "F.Cu") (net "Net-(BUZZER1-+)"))
 (via (at 129 105.5) (size 0.6) (drill 0.3) (layers "F.Cu" "B.Cu") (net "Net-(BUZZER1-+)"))
 (segment (start 129 105.5) (end 134.1 100.4) (width 0.2) (layer "B.Cu") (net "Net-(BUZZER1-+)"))
 (segment (start 134.1 100.4) (end 134.1 86) (width 0.2) (layer "B.Cu") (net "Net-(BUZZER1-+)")))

